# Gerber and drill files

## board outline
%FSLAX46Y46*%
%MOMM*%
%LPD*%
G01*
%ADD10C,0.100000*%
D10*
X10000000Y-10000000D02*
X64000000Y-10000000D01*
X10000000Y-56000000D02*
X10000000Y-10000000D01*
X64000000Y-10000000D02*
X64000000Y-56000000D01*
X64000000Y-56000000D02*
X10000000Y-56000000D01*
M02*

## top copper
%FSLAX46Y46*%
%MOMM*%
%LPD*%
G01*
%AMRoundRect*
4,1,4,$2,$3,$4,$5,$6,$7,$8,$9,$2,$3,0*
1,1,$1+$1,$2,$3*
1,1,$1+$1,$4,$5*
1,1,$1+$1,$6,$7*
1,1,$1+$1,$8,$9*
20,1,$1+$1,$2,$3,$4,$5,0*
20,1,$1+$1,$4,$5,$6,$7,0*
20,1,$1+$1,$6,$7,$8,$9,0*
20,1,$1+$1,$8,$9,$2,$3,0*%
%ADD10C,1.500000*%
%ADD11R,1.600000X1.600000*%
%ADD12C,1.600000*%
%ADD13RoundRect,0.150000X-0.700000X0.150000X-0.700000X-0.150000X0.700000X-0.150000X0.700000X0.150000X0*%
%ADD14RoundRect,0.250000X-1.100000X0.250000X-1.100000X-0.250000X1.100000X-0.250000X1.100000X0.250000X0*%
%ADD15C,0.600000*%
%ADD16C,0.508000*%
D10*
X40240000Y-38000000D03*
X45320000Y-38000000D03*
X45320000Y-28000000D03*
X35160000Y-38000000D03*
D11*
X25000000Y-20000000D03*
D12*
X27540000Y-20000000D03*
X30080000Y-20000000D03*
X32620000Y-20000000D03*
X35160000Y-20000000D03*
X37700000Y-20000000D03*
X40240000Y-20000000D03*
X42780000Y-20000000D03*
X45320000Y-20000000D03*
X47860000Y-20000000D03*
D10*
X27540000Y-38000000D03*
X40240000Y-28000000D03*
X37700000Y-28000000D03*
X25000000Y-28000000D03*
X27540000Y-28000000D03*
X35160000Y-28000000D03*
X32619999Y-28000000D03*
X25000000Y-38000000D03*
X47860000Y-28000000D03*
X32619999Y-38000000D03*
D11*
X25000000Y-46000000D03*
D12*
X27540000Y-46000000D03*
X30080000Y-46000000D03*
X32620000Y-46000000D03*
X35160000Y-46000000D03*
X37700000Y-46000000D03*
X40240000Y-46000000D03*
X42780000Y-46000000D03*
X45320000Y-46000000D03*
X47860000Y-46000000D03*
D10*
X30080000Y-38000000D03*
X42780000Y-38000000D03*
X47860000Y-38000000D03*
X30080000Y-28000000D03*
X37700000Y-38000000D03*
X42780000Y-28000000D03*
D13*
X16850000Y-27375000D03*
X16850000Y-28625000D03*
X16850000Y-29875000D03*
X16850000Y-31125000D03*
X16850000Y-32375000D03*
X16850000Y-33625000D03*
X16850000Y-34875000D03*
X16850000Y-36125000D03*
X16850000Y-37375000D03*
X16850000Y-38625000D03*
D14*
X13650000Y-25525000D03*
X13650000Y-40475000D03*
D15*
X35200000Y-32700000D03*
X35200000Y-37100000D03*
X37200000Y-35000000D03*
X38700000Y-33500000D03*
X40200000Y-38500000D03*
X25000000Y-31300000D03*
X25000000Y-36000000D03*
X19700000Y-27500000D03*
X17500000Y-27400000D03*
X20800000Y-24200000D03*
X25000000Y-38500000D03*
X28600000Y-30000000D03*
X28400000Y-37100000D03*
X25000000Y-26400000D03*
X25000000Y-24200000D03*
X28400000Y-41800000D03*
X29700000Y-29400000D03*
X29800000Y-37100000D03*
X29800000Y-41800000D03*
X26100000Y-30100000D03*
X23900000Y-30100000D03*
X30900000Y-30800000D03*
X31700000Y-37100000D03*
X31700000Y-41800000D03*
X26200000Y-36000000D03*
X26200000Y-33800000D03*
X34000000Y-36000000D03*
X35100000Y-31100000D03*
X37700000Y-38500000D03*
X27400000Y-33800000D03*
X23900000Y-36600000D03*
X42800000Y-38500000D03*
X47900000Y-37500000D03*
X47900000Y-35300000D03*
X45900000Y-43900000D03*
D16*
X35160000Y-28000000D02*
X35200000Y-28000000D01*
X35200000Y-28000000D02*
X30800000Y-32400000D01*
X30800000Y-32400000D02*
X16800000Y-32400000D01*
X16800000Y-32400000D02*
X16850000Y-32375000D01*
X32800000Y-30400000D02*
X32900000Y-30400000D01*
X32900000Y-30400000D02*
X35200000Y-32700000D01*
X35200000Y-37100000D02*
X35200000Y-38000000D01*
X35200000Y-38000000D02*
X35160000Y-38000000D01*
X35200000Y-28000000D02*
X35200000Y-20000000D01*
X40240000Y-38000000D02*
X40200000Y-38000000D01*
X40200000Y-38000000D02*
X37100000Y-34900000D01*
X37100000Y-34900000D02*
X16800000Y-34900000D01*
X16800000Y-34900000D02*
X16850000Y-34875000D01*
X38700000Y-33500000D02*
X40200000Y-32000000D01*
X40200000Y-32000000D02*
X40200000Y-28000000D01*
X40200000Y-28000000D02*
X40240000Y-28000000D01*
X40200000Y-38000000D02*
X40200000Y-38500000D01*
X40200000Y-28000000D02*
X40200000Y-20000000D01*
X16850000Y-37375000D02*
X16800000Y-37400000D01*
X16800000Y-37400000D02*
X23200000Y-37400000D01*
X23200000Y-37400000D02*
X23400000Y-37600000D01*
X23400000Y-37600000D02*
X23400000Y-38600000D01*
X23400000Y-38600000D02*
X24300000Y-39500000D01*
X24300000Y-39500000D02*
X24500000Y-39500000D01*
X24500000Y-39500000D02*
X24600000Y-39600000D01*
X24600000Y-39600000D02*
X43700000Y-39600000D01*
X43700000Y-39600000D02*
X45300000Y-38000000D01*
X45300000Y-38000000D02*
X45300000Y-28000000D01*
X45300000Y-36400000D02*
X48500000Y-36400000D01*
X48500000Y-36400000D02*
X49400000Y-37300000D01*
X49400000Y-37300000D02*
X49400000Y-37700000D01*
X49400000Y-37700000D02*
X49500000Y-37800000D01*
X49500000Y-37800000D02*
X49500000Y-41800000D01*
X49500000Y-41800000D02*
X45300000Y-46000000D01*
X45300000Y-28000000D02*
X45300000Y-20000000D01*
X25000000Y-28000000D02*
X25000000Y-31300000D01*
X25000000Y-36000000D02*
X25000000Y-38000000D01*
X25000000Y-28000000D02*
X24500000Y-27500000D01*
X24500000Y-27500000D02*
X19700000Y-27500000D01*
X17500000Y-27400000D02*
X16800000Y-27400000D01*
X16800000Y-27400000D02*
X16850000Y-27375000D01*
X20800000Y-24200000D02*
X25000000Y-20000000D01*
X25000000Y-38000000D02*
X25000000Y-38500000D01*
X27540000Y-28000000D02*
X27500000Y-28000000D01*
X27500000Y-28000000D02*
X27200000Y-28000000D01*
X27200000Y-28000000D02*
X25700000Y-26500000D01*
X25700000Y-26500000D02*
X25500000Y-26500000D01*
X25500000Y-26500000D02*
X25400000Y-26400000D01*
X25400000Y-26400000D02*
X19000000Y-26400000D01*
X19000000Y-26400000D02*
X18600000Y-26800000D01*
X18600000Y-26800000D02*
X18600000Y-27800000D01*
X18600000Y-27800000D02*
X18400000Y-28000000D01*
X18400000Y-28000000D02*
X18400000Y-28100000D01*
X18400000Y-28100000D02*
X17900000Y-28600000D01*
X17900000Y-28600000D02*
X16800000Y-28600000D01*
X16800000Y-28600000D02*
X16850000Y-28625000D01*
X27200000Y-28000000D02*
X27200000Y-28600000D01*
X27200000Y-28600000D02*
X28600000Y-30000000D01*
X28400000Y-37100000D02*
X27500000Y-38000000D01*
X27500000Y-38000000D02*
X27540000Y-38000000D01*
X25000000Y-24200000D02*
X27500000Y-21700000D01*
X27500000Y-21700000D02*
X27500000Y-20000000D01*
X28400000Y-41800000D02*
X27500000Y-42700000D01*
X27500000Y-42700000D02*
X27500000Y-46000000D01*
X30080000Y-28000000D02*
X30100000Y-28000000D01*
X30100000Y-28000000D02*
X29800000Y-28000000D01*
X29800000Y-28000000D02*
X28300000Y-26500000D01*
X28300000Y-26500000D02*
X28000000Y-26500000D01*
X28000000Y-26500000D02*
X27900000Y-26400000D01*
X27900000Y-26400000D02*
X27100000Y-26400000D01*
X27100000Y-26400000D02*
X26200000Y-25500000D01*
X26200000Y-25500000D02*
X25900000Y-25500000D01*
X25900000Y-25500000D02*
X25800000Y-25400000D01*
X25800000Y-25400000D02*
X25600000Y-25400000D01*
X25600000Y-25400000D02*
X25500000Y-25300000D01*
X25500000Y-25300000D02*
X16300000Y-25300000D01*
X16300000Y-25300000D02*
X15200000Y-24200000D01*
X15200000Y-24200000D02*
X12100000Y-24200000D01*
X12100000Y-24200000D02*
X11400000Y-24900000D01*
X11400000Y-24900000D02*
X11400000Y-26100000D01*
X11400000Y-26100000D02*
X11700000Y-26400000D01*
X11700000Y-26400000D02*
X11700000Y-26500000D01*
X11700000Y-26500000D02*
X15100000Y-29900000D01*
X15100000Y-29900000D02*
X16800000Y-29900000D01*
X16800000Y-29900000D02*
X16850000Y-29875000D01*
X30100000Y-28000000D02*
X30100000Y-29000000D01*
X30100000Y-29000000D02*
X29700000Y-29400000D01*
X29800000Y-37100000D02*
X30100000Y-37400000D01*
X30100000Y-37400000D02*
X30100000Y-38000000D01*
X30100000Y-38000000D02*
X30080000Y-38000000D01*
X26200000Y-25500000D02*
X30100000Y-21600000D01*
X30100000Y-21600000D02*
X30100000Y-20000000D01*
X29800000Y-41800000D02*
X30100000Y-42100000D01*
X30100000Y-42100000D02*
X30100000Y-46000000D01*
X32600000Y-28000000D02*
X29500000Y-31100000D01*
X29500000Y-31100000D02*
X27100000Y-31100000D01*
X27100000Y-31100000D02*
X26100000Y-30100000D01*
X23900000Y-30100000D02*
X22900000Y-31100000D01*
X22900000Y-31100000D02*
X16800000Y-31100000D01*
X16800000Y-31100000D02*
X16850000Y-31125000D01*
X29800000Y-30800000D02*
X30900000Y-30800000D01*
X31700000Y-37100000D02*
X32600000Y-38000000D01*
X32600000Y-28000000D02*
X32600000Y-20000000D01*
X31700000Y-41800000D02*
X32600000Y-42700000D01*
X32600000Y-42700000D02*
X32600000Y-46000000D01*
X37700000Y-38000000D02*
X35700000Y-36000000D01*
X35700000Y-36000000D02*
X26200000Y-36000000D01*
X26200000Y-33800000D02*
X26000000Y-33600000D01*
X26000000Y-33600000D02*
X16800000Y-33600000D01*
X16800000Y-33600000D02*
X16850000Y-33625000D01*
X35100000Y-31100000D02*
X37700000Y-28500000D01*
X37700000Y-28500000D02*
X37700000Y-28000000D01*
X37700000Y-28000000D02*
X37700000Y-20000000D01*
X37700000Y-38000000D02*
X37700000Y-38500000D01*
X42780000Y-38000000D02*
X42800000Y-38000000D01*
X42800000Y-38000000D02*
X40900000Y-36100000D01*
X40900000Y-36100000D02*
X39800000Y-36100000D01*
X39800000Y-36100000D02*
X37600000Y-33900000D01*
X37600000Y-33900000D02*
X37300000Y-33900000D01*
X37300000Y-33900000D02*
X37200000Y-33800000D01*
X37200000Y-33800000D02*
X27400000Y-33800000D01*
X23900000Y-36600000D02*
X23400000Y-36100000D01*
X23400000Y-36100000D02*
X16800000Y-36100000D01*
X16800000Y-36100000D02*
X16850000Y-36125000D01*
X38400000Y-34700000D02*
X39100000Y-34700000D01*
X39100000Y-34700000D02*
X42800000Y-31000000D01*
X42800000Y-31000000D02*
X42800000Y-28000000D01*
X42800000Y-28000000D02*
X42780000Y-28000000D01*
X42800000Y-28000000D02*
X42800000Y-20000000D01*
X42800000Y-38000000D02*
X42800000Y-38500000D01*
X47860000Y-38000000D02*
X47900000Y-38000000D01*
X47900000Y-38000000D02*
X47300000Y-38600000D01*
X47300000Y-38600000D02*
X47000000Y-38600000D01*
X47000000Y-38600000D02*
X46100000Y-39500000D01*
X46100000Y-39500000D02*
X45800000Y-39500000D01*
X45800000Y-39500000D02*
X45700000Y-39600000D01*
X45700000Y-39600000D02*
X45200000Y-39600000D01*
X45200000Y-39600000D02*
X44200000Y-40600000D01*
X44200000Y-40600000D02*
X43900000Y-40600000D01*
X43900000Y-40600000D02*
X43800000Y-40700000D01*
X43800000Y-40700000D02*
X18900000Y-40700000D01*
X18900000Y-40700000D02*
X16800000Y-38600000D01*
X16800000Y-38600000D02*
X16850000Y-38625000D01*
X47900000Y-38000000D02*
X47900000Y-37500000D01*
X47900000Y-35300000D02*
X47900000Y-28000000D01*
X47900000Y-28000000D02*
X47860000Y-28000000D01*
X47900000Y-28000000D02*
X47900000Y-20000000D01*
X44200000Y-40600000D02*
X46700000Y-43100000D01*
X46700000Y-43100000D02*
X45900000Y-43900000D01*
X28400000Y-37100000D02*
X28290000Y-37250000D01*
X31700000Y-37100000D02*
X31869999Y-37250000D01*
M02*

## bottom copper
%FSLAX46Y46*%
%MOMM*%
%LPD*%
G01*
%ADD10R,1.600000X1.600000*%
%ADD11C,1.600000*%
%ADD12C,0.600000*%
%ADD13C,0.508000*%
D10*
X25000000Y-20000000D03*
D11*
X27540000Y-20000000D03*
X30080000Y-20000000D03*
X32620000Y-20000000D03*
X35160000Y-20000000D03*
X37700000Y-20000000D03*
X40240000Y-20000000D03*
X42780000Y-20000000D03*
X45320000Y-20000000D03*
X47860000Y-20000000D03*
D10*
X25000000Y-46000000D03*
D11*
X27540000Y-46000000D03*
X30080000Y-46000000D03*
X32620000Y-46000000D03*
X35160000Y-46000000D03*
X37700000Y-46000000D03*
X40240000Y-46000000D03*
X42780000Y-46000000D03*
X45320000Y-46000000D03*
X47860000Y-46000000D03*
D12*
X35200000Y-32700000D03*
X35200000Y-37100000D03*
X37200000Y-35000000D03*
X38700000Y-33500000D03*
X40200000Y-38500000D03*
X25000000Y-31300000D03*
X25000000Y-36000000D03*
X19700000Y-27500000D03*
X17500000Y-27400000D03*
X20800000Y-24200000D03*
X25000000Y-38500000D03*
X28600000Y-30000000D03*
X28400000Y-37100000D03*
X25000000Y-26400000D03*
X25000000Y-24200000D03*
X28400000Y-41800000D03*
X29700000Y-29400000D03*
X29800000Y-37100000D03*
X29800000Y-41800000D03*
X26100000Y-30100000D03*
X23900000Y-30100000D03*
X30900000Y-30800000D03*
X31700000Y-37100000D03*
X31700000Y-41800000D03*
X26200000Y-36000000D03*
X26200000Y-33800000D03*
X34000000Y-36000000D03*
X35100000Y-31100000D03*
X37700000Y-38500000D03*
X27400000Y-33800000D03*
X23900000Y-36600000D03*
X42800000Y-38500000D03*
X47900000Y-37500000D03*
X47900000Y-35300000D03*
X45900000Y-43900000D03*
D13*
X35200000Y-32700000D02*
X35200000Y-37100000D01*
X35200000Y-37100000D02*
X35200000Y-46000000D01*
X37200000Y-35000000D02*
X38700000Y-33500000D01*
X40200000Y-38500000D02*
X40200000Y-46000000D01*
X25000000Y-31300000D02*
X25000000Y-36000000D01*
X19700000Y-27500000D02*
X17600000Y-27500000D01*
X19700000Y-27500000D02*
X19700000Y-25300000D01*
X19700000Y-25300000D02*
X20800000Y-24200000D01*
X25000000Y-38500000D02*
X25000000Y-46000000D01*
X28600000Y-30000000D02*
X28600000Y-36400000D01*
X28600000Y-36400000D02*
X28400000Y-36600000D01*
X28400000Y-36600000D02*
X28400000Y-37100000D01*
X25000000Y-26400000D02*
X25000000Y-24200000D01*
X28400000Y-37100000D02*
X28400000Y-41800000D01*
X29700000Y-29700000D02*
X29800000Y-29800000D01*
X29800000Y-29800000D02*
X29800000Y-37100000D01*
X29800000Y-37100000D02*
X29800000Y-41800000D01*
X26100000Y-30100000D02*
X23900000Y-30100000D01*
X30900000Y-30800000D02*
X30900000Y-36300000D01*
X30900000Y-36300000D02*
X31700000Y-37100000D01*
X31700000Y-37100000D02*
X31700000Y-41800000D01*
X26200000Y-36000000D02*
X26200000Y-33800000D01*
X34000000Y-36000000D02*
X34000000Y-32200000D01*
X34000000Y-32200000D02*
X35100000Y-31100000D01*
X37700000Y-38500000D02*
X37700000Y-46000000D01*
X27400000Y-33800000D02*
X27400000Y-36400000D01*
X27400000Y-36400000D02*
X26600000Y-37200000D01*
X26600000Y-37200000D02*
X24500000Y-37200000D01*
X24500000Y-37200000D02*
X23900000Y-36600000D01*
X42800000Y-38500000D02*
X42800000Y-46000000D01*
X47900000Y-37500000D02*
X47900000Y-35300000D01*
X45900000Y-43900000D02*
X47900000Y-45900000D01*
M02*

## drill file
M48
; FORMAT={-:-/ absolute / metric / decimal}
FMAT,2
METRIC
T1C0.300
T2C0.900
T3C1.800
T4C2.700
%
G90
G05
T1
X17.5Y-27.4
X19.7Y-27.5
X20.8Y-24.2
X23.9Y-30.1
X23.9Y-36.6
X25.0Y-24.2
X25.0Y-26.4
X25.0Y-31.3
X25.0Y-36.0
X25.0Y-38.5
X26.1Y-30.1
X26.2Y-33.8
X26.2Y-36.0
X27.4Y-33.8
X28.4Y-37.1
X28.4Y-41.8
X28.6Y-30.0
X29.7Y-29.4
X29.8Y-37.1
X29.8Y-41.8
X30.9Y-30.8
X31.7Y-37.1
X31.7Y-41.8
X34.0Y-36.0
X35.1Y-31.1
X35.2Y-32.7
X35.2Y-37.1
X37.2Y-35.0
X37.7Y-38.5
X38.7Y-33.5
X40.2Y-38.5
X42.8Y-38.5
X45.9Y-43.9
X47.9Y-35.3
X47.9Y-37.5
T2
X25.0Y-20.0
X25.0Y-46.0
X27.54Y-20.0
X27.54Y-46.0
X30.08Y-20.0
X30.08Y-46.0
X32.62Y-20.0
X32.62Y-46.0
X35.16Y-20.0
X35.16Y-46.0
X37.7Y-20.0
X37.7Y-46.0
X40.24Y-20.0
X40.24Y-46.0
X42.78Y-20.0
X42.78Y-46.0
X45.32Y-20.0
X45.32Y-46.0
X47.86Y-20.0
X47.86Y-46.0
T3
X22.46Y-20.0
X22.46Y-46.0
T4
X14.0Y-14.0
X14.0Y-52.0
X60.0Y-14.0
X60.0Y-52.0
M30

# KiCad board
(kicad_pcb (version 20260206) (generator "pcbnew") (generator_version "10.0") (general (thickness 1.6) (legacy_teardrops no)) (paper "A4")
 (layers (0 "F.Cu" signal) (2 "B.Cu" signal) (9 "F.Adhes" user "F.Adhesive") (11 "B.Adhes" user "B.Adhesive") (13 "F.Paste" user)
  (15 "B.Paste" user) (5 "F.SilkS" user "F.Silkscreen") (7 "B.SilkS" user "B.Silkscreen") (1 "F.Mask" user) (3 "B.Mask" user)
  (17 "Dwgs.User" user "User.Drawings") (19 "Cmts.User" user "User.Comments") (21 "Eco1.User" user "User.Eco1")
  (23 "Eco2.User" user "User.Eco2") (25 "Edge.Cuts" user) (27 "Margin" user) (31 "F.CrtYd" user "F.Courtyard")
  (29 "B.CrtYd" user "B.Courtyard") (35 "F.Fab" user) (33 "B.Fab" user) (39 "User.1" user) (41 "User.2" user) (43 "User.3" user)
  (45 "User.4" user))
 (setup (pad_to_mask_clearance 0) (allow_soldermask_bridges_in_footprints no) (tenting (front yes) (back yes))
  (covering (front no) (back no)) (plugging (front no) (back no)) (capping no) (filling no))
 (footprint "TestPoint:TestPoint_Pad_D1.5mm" (layer "F.Cu") (at 40.24 38)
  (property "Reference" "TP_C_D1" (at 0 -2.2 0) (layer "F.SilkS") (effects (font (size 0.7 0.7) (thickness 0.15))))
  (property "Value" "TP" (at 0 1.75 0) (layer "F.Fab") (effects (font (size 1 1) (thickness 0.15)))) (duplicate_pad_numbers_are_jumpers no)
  (pad "1" smd circle (at 0 0) (size 1.5 1.5) (layers "F.Cu" "F.Mask") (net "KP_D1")))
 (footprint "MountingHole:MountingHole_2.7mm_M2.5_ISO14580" (layer "F.Cu") (at 60 14)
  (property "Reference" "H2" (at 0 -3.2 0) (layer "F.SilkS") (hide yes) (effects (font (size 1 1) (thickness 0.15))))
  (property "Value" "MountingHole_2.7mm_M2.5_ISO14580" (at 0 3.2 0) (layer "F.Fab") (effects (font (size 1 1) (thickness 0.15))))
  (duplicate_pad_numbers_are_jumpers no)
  (pad "" np_thru_hole circle (at 0 0) (size 2.7 2.7) (drill 2.7) (layers "*.Cu" "*.Mask")))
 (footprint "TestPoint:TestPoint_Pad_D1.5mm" (layer "F.Cu") (at 45.32 38)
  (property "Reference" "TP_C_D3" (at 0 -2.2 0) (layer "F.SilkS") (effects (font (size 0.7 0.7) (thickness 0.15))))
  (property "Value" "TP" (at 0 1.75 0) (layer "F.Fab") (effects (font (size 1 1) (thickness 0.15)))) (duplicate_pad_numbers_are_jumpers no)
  (pad "1" smd circle (at 0 0) (size 1.5 1.5) (layers "F.Cu" "F.Mask") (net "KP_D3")))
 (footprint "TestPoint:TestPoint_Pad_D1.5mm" (layer "F.Cu") (at 45.32 28)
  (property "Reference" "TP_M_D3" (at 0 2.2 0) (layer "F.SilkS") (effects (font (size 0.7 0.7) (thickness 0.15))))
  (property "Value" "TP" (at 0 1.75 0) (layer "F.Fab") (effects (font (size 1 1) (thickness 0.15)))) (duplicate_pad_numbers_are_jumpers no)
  (pad "1" smd circle (at 0 0) (size 1.5 1.5) (layers "F.Cu" "F.Mask") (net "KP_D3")))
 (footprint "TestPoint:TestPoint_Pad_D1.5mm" (layer "F.Cu") (at 35.16 38)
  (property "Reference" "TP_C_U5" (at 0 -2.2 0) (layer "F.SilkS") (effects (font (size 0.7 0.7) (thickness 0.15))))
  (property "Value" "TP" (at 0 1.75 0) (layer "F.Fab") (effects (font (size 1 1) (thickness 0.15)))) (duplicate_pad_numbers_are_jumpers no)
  (pad "1" smd circle (at 0 0) (size 1.5 1.5) (layers "F.Cu" "F.Mask") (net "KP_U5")))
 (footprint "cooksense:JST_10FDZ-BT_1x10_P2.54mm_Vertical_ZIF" (layer "F.Cu") (at 25 20)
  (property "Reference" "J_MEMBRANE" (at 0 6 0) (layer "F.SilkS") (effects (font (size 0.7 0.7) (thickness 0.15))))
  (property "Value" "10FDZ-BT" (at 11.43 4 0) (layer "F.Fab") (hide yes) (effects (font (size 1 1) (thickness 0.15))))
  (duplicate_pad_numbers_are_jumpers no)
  (pad "" np_thru_hole circle (at -2.54 0) (size 1.8 1.8) (drill 1.8) (layers "*.Cu" "*.Mask"))
  (pad "1" thru_hole rect (at 0 0) (size 1.6 1.6) (drill 0.9) (layers "*.Cu" "*.Mask") (remove_unused_layers no) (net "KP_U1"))
  (pad "2" thru_hole circle (at 2.54 0) (size 1.6 1.6) (drill 0.9) (layers "*.Cu" "*.Mask") (remove_unused_layers no) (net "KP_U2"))
  (pad "3" thru_hole circle (at 5.08 0) (size 1.6 1.6) (drill 0.9) (layers "*.Cu" "*.Mask") (remove_unused_layers no) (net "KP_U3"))
  (pad "4" thru_hole circle (at 7.62 0) (size 1.6 1.6) (drill 0.9) (layers "*.Cu" "*.Mask") (remove_unused_layers no) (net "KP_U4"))
  (pad "5" thru_hole circle (at 10.16 0) (size 1.6 1.6) (drill 0.9) (layers "*.Cu" "*.Mask") (remove_unused_layers no) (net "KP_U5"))
  (pad "6" thru_hole circle (at 12.7 0) (size 1.6 1.6) (drill 0.9) (layers "*.Cu" "*.Mask") (remove_unused_layers no) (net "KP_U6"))
  (pad "7" thru_hole circle (at 15.24 0) (size 1.6 1.6) (drill 0.9) (layers "*.Cu" "*.Mask") (remove_unused_layers no) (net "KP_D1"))
  (pad "8" thru_hole circle (at 17.78 0) (size 1.6 1.6) (drill 0.9) (layers "*.Cu" "*.Mask") (remove_unused_layers no) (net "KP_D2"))
  (pad "9" thru_hole circle (at 20.32 0) (size 1.6 1.6) (drill 0.9) (layers "*.Cu" "*.Mask") (remove_unused_layers no) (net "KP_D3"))
  (pad "10" thru_hole circle (at 22.86 0) (size 1.6 1.6) (drill 0.9) (layers "*.Cu" "*.Mask") (remove_unused_layers no) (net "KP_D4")))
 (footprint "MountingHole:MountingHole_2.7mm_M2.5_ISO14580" (layer "F.Cu") (at 14 14)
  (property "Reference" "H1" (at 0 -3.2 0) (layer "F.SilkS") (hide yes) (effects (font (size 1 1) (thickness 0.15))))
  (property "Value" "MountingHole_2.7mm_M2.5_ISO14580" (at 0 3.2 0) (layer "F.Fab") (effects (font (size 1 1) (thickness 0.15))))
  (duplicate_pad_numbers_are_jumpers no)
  (pad "" np_thru_hole circle (at 0 0) (size 2.7 2.7) (drill 2.7) (layers "*.Cu" "*.Mask")))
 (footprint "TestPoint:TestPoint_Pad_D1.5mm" (layer "F.Cu") (at 27.54 38)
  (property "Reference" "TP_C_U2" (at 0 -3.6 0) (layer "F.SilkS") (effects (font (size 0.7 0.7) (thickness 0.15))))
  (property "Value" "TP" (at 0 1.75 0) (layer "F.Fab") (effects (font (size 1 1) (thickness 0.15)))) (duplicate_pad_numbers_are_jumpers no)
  (pad "1" smd circle (at 0 0) (size 1.5 1.5) (layers "F.Cu" "F.Mask") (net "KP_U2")))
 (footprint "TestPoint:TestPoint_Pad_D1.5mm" (layer "F.Cu") (at 40.24 28)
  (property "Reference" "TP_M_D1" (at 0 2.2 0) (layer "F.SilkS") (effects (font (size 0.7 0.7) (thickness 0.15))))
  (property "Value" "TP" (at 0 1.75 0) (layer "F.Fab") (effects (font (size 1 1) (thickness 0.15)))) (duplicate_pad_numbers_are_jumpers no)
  (pad "1" smd circle (at 0 0) (size 1.5 1.5) (layers "F.Cu" "F.Mask") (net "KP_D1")))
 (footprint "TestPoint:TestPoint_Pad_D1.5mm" (layer "F.Cu") (at 37.7 28)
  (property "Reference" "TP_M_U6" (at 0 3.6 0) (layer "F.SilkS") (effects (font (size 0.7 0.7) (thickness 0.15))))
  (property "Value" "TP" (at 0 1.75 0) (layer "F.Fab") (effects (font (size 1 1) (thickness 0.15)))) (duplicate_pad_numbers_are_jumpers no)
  (pad "1" smd circle (at 0 0) (size 1.5 1.5) (layers "F.Cu" "F.Mask") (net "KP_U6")))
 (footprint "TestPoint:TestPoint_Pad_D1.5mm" (layer "F.Cu") (at 25 28)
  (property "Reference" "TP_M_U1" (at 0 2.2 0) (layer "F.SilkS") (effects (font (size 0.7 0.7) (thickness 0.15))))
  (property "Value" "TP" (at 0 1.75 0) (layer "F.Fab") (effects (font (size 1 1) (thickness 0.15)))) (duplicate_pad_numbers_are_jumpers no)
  (pad "1" smd circle (at 0 0) (size 1.5 1.5) (layers "F.Cu" "F.Mask") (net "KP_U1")))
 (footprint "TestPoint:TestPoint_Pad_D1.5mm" (layer "F.Cu") (at 27.54 28)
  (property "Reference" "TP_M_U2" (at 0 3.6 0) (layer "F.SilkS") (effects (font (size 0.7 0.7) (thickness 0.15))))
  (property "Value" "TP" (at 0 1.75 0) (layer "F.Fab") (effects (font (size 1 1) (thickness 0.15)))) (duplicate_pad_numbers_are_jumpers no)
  (pad "1" smd circle (at 0 0) (size 1.5 1.5) (layers "F.Cu" "F.Mask") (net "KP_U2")))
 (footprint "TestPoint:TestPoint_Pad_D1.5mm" (layer "F.Cu") (at 35.16 28)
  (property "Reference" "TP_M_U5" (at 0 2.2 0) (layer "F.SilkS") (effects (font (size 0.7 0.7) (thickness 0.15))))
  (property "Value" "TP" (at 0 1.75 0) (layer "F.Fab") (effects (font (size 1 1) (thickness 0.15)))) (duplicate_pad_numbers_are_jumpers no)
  (pad "1" smd circle (at 0 0) (size 1.5 1.5) (layers "F.Cu" "F.Mask") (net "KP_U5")))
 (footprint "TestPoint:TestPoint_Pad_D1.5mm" (layer "F.Cu") (at 32.619999 28)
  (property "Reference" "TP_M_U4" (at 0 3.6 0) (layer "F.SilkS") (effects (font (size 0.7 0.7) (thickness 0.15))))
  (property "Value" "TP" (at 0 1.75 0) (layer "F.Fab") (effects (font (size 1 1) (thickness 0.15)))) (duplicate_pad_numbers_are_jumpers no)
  (pad "1" smd circle (at 0 0) (size 1.5 1.5) (layers "F.Cu" "F.Mask") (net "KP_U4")))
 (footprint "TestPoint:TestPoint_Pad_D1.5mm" (layer "F.Cu") (at 25 38)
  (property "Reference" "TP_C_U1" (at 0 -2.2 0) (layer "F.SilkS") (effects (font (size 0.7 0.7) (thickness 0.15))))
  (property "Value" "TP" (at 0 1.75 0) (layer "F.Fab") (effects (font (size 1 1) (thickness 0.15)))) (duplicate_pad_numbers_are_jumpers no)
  (pad "1" smd circle (at 0 0) (size 1.5 1.5) (layers "F.Cu" "F.Mask") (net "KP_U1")))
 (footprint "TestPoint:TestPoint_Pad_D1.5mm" (layer "F.Cu") (at 47.86 28)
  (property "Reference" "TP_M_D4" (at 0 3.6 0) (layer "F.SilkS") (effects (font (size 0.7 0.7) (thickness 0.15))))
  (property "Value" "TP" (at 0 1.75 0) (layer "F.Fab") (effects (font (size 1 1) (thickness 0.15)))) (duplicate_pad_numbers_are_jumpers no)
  (pad "1" smd circle (at 0 0) (size 1.5 1.5) (layers "F.Cu" "F.Mask") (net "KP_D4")))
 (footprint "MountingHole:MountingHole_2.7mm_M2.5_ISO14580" (layer "F.Cu") (at 60 52)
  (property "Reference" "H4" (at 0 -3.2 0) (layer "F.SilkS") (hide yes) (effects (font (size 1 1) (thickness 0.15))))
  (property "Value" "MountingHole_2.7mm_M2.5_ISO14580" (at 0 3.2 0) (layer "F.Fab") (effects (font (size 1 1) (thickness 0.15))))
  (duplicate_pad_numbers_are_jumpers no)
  (pad "" np_thru_hole circle (at 0 0) (size 2.7 2.7) (drill 2.7) (layers "*.Cu" "*.Mask")))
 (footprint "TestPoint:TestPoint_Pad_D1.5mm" (layer "F.Cu") (at 32.619999 38)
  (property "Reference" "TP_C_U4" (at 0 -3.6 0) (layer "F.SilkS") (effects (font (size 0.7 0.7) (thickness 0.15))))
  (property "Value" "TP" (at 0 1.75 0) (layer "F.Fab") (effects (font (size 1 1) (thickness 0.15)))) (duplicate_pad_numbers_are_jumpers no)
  (pad "1" smd circle (at 0 0) (size 1.5 1.5) (layers "F.Cu" "F.Mask") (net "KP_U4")))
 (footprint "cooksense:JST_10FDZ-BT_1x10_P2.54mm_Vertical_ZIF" (layer "F.Cu") (at 25 46)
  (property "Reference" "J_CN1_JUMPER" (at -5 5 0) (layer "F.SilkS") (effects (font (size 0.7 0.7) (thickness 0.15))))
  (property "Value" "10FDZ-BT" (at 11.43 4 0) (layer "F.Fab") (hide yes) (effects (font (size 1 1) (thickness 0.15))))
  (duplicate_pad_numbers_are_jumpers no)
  (pad "" np_thru_hole circle (at -2.54 0) (size 1.8 1.8) (drill 1.8) (layers "*.Cu" "*.Mask"))
  (pad "1" thru_hole rect (at 0 0) (size 1.6 1.6) (drill 0.9) (layers "*.Cu" "*.Mask") (remove_unused_layers no) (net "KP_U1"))
  (pad "2" thru_hole circle (at 2.54 0) (size 1.6 1.6) (drill 0.9) (layers "*.Cu" "*.Mask") (remove_unused_layers no) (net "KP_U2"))
  (pad "3" thru_hole circle (at 5.08 0) (size 1.6 1.6) (drill 0.9) (layers "*.Cu" "*.Mask") (remove_unused_layers no) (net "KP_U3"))
  (pad "4" thru_hole circle (at 7.62 0) (size 1.6 1.6) (drill 0.9) (layers "*.Cu" "*.Mask") (remove_unused_layers no) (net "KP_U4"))
  (pad "5" thru_hole circle (at 10.16 0) (size 1.6 1.6) (drill 0.9) (layers "*.Cu" "*.Mask") (remove_unused_layers no) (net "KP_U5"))
  (pad "6" thru_hole circle (at 12.7 0) (size 1.6 1.6) (drill 0.9) (layers "*.Cu" "*.Mask") (remove_unused_layers no) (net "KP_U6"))
  (pad "7" thru_hole circle (at 15.24 0) (size 1.6 1.6) (drill 0.9) (layers "*.Cu" "*.Mask") (remove_unused_layers no) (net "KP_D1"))
  (pad "8" thru_hole circle (at 17.78 0) (size 1.6 1.6) (drill 0.9) (layers "*.Cu" "*.Mask") (remove_unused_layers no) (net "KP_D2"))
  (pad "9" thru_hole circle (at 20.32 0) (size 1.6 1.6) (drill 0.9) (layers "*.Cu" "*.Mask") (remove_unused_layers no) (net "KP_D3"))
  (pad "10" thru_hole circle (at 22.86 0) (size 1.6 1.6) (drill 0.9) (layers "*.Cu" "*.Mask") (remove_unused_layers no) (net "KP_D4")))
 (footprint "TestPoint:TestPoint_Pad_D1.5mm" (layer "F.Cu") (at 30.08 38)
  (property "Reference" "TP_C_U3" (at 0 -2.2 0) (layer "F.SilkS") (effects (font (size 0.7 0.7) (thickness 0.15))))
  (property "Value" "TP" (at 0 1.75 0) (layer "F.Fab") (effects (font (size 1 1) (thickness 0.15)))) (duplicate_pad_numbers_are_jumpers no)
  (pad "1" smd circle (at 0 0) (size 1.5 1.5) (layers "F.Cu" "F.Mask") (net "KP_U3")))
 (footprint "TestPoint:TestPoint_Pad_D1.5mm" (layer "F.Cu") (at 42.78 38)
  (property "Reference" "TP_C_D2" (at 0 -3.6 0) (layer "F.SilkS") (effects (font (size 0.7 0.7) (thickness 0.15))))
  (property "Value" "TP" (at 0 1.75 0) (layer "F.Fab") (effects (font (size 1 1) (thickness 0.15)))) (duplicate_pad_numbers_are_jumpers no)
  (pad "1" smd circle (at 0 0) (size 1.5 1.5) (layers "F.Cu" "F.Mask") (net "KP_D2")))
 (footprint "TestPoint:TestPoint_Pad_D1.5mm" (layer "F.Cu") (at 47.86 38)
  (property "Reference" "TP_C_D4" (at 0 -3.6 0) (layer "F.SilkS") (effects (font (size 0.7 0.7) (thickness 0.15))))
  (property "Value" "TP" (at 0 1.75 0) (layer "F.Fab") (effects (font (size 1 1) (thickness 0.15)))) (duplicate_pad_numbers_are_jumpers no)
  (pad "1" smd circle (at 0 0) (size 1.5 1.5) (layers "F.Cu" "F.Mask") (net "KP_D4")))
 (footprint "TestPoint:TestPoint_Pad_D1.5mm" (layer "F.Cu") (at 30.08 28)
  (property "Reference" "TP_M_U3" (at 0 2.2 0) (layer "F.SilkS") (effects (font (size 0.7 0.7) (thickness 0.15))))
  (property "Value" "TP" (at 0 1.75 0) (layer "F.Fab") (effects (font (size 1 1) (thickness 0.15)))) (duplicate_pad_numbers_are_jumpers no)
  (pad "1" smd circle (at 0 0) (size 1.5 1.5) (layers "F.Cu" "F.Mask") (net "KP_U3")))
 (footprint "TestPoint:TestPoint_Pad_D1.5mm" (layer "F.Cu") (at 37.7 38)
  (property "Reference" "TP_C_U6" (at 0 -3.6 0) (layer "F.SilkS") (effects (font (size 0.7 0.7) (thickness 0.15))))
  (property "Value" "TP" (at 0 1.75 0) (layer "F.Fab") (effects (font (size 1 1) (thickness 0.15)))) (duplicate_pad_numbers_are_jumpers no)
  (pad "1" smd circle (at 0 0) (size 1.5 1.5) (layers "F.Cu" "F.Mask") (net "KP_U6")))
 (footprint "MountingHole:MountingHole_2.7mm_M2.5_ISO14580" (layer "F.Cu") (at 14 52)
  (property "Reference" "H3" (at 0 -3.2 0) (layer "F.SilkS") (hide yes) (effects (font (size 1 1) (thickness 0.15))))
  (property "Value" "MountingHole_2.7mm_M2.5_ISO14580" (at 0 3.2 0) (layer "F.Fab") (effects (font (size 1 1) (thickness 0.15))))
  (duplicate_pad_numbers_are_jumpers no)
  (pad "" np_thru_hole circle (at 0 0) (size 2.7 2.7) (drill 2.7) (layers "*.Cu" "*.Mask")))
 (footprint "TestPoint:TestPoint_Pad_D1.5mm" (layer "F.Cu") (at 42.78 28)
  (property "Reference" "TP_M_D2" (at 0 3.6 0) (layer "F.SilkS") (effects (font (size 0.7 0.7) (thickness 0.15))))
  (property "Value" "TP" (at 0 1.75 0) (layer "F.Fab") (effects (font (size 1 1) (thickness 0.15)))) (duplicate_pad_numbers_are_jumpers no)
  (pad "1" smd circle (at 0 0) (size 1.5 1.5) (layers "F.Cu" "F.Mask") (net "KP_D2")))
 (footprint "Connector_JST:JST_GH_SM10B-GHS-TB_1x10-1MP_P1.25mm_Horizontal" (layer "F.Cu") (at 15 33 -90)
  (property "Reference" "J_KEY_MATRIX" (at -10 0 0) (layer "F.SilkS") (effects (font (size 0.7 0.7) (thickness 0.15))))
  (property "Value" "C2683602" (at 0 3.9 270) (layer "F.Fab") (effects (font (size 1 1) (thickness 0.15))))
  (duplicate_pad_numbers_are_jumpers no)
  (pad "1" smd roundrect (at -5.625 -1.85 270) (size 0.6 1.7) (layers "F.Cu" "F.Mask" "F.Paste") (roundrect_rratio 0.25) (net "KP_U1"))
  (pad "2" smd roundrect (at -4.375 -1.85 270) (size 0.6 1.7) (layers "F.Cu" "F.Mask" "F.Paste") (roundrect_rratio 0.25) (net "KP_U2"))
  (pad "3" smd roundrect (at -3.125 -1.85 270) (size 0.6 1.7) (layers "F.Cu" "F.Mask" "F.Paste") (roundrect_rratio 0.25) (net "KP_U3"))
  (pad "4" smd roundrect (at -1.875 -1.85 270) (size 0.6 1.7) (layers "F.Cu" "F.Mask" "F.Paste") (roundrect_rratio 0.25) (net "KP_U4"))
  (pad "5" smd roundrect (at -0.625 -1.85 270) (size 0.6 1.7) (layers "F.Cu" "F.Mask" "F.Paste") (roundrect_rratio 0.25) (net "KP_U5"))
  (pad "6" smd roundrect (at 0.625 -1.85 270) (size 0.6 1.7) (layers "F.Cu" "F.Mask" "F.Paste") (roundrect_rratio 0.25) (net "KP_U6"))
  (pad "7" smd roundrect (at 1.875 -1.85 270) (size 0.6 1.7) (layers "F.Cu" "F.Mask" "F.Paste") (roundrect_rratio 0.25) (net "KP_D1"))
  (pad "8" smd roundrect (at 3.125 -1.85 270) (size 0.6 1.7) (layers "F.Cu" "F.Mask" "F.Paste") (roundrect_rratio 0.25) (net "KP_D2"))
  (pad "9" smd roundrect (at 4.375 -1.85 270) (size 0.6 1.7) (layers "F.Cu" "F.Mask" "F.Paste") (roundrect_rratio 0.25) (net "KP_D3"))
  (pad "10" smd roundrect (at 5.625 -1.85 270) (size 0.6 1.7) (layers "F.Cu" "F.Mask" "F.Paste") (roundrect_rratio 0.25) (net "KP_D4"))
  (pad "MP" smd roundrect (at -7.475 1.35 270) (size 1 2.7) (layers "F.Cu" "F.Mask" "F.Paste") (roundrect_rratio 0.25))
  (pad "MP" smd roundrect (at 7.475 1.35 270) (size 1 2.7) (layers "F.Cu" "F.Mask" "F.Paste") (roundrect_rratio 0.25)))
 (gr_line (start 10 10) (end 64 10) (stroke (width 0.1) (type default)) (layer "Edge.Cuts"))
 (gr_line (start 10 56) (end 10 10) (stroke (width 0.1) (type default)) (layer "Edge.Cuts"))
 (gr_line (start 64 10) (end 64 56) (stroke (width 0.1) (type default)) (layer "Edge.Cuts"))
 (gr_line (start 64 56) (end 10 56) (stroke (width 0.1) (type default)) (layer "Edge.Cuts"))
 (segment (start 35.160000 28.000000) (end 35.200000 28.000000) (width 0.508) (layer "F.Cu") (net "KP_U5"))
 (segment (start 35.200000 28.000000) (end 30.800000 32.400000) (width 0.508) (layer "F.Cu") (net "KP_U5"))
 (segment (start 30.800000 32.400000) (end 16.800000 32.400000) (width 0.508) (layer "F.Cu") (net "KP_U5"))
 (segment (start 16.800000 32.400000) (end 16.850000 32.375000) (width 0.508) (layer "F.Cu") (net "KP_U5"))
 (segment (start 32.800000 30.400000) (end 32.900000 30.400000) (width 0.508) (layer "F.Cu") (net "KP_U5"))
 (segment (start 32.900000 30.400000) (end 35.200000 32.700000) (width 0.508) (layer "F.Cu") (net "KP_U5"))
 (segment (start 35.200000 32.700000) (end 35.200000 37.100000) (width 0.508) (layer "B.Cu") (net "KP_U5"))
 (segment (start 35.200000 37.100000) (end 35.200000 38.000000) (width 0.508) (layer "F.Cu") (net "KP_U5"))
 (segment (start 35.200000 38.000000) (end 35.160000 38.000000) (width 0.508) (layer "F.Cu") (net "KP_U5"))
 (segment (start 35.200000 37.100000) (end 35.200000 46.000000) (width 0.508) (layer "B.Cu") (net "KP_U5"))
 (segment (start 35.200000 28.000000) (end 35.200000 20.000000) (width 0.508) (layer "F.Cu") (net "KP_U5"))
 (via (at 35.200000 32.700000) (size 0.6) (drill 0.3) (layers "F.Cu" "B.Cu") (tenting (front yes) (back yes)) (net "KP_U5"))
 (via (at 35.200000 37.100000) (size 0.6) (drill 0.3) (layers "F.Cu" "B.Cu") (tenting (front yes) (back yes)) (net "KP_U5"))
 (segment (start 40.240000 38.000000) (end 40.200000 38.000000) (width 0.508) (layer "F.Cu") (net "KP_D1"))
 (segment (start 40.200000 38.000000) (end 37.100000 34.900000) (width 0.508) (layer "F.Cu") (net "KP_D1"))
 (segment (start 37.100000 34.900000) (end 16.800000 34.900000) (width 0.508) (layer "F.Cu") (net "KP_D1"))
 (segment (start 16.800000 34.900000) (end 16.850000 34.875000) (width 0.508) (layer "F.Cu") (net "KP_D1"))
 (segment (start 37.200000 35.000000) (end 38.700000 33.500000) (width 0.508) (layer "B.Cu") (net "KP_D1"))
 (segment (start 38.700000 33.500000) (end 40.200000 32.000000) (width 0.508) (layer "F.Cu") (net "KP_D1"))
 (segment (start 40.200000 32.000000) (end 40.200000 28.000000) (width 0.508) (layer "F.Cu") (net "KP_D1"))
 (segment (start 40.200000 28.000000) (end 40.240000 28.000000) (width 0.508) (layer "F.Cu") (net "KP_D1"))
 (segment (start 40.200000 38.000000) (end 40.200000 38.500000) (width 0.508) (layer "F.Cu") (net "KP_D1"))
 (segment (start 40.200000 38.500000) (end 40.200000 46.000000) (width 0.508) (layer "B.Cu") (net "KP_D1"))
 (segment (start 40.200000 28.000000) (end 40.200000 20.000000) (width 0.508) (layer "F.Cu") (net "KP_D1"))
 (via (at 37.200000 35.000000) (size 0.6) (drill 0.3) (layers "F.Cu" "B.Cu") (tenting (front yes) (back yes)) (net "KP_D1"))
 (via (at 38.700000 33.500000) (size 0.6) (drill 0.3) (layers "F.Cu" "B.Cu") (tenting (front yes) (back yes)) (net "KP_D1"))
 (via (at 40.200000 38.500000) (size 0.6) (drill 0.3) (layers "F.Cu" "B.Cu") (tenting (front yes) (back yes)) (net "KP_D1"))
 (segment (start 16.850000 37.375000) (end 16.800000 37.400000) (width 0.508) (layer "F.Cu") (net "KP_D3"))
 (segment (start 16.800000 37.400000) (end 23.200000 37.400000) (width 0.508) (layer "F.Cu") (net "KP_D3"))
 (segment (start 23.200000 37.400000) (end 23.400000 37.600000) (width 0.508) (layer "F.Cu") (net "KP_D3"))
 (segment (start 23.400000 37.600000) (end 23.400000 38.600000) (width 0.508) (layer "F.Cu") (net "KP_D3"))
 (segment (start 23.400000 38.600000) (end 24.300000 39.500000) (width 0.508) (layer "F.Cu") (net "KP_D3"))
 (segment (start 24.300000 39.500000) (end 24.500000 39.500000) (width 0.508) (layer "F.Cu") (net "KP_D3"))
 (segment (start 24.500000 39.500000) (end 24.600000 39.600000) (width 0.508) (layer "F.Cu") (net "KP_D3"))
 (segment (start 24.600000 39.600000) (end 43.700000 39.600000) (width 0.508) (layer "F.Cu") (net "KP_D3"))
 (segment (start 43.700000 39.600000) (end 45.300000 38.000000) (width 0.508) (layer "F.Cu") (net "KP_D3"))
 (segment (start 45.300000 38.000000) (end 45.300000 28.000000) (width 0.508) (layer "F.Cu") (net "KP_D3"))
 (segment (start 45.300000 36.400000) (end 48.500000 36.400000) (width 0.508) (layer "F.Cu") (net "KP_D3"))
 (segment (start 48.500000 36.400000) (end 49.400000 37.300000) (width 0.508) (layer "F.Cu") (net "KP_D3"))
 (segment (start 49.400000 37.300000) (end 49.400000 37.700000) (width 0.508) (layer "F.Cu") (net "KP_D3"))
 (segment (start 49.400000 37.700000) (end 49.500000 37.800000) (width 0.508) (layer "F.Cu") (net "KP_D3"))
 (segment (start 49.500000 37.800000) (end 49.500000 41.800000) (width 0.508) (layer "F.Cu") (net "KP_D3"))
 (segment (start 49.500000 41.800000) (end 45.300000 46.000000) (width 0.508) (layer "F.Cu") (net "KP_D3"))
 (segment (start 45.300000 28.000000) (end 45.300000 20.000000) (width 0.508) (layer "F.Cu") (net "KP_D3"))
 (segment (start 25.000000 28.000000) (end 25.000000 31.300000) (width 0.508) (layer "F.Cu") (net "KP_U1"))
 (segment (start 25.000000 31.300000) (end 25.000000 36.000000) (width 0.508) (layer "B.Cu") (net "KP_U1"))
 (segment (start 25.000000 36.000000) (end 25.000000 38.000000) (width 0.508) (layer "F.Cu") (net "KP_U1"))
 (segment (start 25.000000 28.000000) (end 24.500000 27.500000) (width 0.508) (layer "F.Cu") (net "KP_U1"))
 (segment (start 24.500000 27.500000) (end 19.700000 27.500000) (width 0.508) (layer "F.Cu") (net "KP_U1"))
 (segment (start 19.700000 27.500000) (end 17.600000 27.500000) (width 0.508) (layer "B.Cu") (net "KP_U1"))
 (segment (start 17.500000 27.400000) (end 16.800000 27.400000) (width 0.508) (layer "F.Cu") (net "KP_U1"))
 (segment (start 16.800000 27.400000) (end 16.850000 27.375000) (width 0.508) (layer "F.Cu") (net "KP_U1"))
 (segment (start 19.700000 27.500000) (end 19.700000 25.300000) (width 0.508) (layer "B.Cu") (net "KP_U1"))
 (segment (start 19.700000 25.300000) (end 20.800000 24.200000) (width 0.508) (layer "B.Cu") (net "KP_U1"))
 (segment (start 20.800000 24.200000) (end 25.000000 20.000000) (width 0.508) (layer "F.Cu") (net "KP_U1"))
 (segment (start 25.000000 38.000000) (end 25.000000 38.500000) (width 0.508) (layer "F.Cu") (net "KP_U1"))
 (segment (start 25.000000 38.500000) (end 25.000000 46.000000) (width 0.508) (layer "B.Cu") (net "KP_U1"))
 (via (at 25.000000 31.300000) (size 0.6) (drill 0.3) (layers "F.Cu" "B.Cu") (tenting (front yes) (back yes)) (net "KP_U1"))
 (via (at 25.000000 36.000000) (size 0.6) (drill 0.3) (layers "F.Cu" "B.Cu") (tenting (front yes) (back yes)) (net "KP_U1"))
 (via (at 19.700000 27.500000) (size 0.6) (drill 0.3) (layers "F.Cu" "B.Cu") (tenting (front yes) (back yes)) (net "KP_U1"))
 (via (at 17.500000 27.400000) (size 0.6) (drill 0.3) (layers "F.Cu" "B.Cu") (tenting (front yes) (back yes)) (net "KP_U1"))
 (via (at 20.800000 24.200000) (size 0.6) (drill 0.3) (layers "F.Cu" "B.Cu") (tenting (front yes) (back yes)) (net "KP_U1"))
 (via (at 25.000000 38.500000) (size 0.6) (drill 0.3) (layers "F.Cu" "B.Cu") (tenting (front yes) (back yes)) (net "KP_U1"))
 (segment (start 27.540000 28.000000) (end 27.500000 28.000000) (width 0.508) (layer "F.Cu") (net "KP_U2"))
 (segment (start 27.500000 28.000000) (end 27.200000 28.000000) (width 0.508) (layer "F.Cu") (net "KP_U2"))
 (segment (start 27.200000 28.000000) (end 25.700000 26.500000) (width 0.508) (layer "F.Cu") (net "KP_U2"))
 (segment (start 25.700000 26.500000) (end 25.500000 26.500000) (width 0.508) (layer "F.Cu") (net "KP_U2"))
 (segment (start 25.500000 26.500000) (end 25.400000 26.400000) (width 0.508) (layer "F.Cu") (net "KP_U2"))
 (segment (start 25.400000 26.400000) (end 19.000000 26.400000) (width 0.508) (layer "F.Cu") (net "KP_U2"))
 (segment (start 19.000000 26.400000) (end 18.600000 26.800000) (width 0.508) (layer "F.Cu") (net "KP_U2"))
 (segment (start 18.600000 26.800000) (end 18.600000 27.800000) (width 0.508) (layer "F.Cu") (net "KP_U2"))
 (segment (start 18.600000 27.800000) (end 18.400000 28.000000) (width 0.508) (layer "F.Cu") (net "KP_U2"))
 (segment (start 18.400000 28.000000) (end 18.400000 28.100000) (width 0.508) (layer "F.Cu") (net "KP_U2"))
 (segment (start 18.400000 28.100000) (end 17.900000 28.600000) (width 0.508) (layer "F.Cu") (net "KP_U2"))
 (segment (start 17.900000 28.600000) (end 16.800000 28.600000) (width 0.508) (layer "F.Cu") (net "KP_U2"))
 (segment (start 16.800000 28.600000) (end 16.850000 28.625000) (width 0.508) (layer "F.Cu") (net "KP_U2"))
 (segment (start 27.200000 28.000000) (end 27.200000 28.600000) (width 0.508) (layer "F.Cu") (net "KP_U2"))
 (segment (start 27.200000 28.600000) (end 28.600000 30.000000) (width 0.508) (layer "F.Cu") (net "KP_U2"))
 (segment (start 28.600000 30.000000) (end 28.600000 36.400000) (width 0.508) (layer "B.Cu") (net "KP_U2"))
 (segment (start 28.600000 36.400000) (end 28.400000 36.600000) (width 0.508) (layer "B.Cu") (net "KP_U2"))
 (segment (start 28.400000 36.600000) (end 28.400000 37.100000) (width 0.508) (layer "B.Cu") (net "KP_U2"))
 (segment (start 28.400000 37.100000) (end 27.500000 38.000000) (width 0.508) (layer "F.Cu") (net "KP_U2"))
 (segment (start 27.500000 38.000000) (end 27.540000 38.000000) (width 0.508) (layer "F.Cu") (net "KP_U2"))
 (segment (start 25.000000 26.400000) (end 25.000000 24.200000) (width 0.508) (layer "B.Cu") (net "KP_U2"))
 (segment (start 25.000000 24.200000) (end 27.500000 21.700000) (width 0.508) (layer "F.Cu") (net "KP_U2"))
 (segment (start 27.500000 21.700000) (end 27.500000 20.000000) (width 0.508) (layer "F.Cu") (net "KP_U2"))
 (segment (start 28.400000 37.100000) (end 28.400000 41.800000) (width 0.508) (layer "B.Cu") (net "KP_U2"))
 (segment (start 28.400000 41.800000) (end 27.500000 42.700000) (width 0.508) (layer "F.Cu") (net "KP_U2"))
 (segment (start 27.500000 42.700000) (end 27.500000 46.000000) (width 0.508) (layer "F.Cu") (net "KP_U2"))
 (via (at 28.600000 30.000000) (size 0.6) (drill 0.3) (layers "F.Cu" "B.Cu") (tenting (front yes) (back yes)) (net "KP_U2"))
 (via (at 28.400000 37.100000) (size 0.6) (drill 0.3) (layers "F.Cu" "B.Cu") (tenting (front yes) (back yes)) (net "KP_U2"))
 (via (at 25.000000 26.400000) (size 0.6) (drill 0.3) (layers "F.Cu" "B.Cu") (tenting (front yes) (back yes)) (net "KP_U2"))
 (via (at 25.000000 24.200000) (size 0.6) (drill 0.3) (layers "F.Cu" "B.Cu") (tenting (front yes) (back yes)) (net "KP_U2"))
 (via (at 28.400000 41.800000) (size 0.6) (drill 0.3) (layers "F.Cu" "B.Cu") (tenting (front yes) (back yes)) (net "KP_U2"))
 (segment (start 30.080000 28.000000) (end 30.100000 28.000000) (width 0.508) (layer "F.Cu") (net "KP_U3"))
 (segment (start 30.100000 28.000000) (end 29.800000 28.000000) (width 0.508) (layer "F.Cu") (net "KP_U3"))
 (segment (start 29.800000 28.000000) (end 28.300000 26.500000) (width 0.508) (layer "F.Cu") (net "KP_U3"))
 (segment (start 28.300000 26.500000) (end 28.000000 26.500000) (width 0.508) (layer "F.Cu") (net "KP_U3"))
 (segment (start 28.000000 26.500000) (end 27.900000 26.400000) (width 0.508) (layer "F.Cu") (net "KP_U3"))
 (segment (start 27.900000 26.400000) (end 27.100000 26.400000) (width 0.508) (layer "F.Cu") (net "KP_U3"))
 (segment (start 27.100000 26.400000) (end 26.200000 25.500000) (width 0.508) (layer "F.Cu") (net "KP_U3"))
 (segment (start 26.200000 25.500000) (end 25.900000 25.500000) (width 0.508) (layer "F.Cu") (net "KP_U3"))
 (segment (start 25.900000 25.500000) (end 25.800000 25.400000) (width 0.508) (layer "F.Cu") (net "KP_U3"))
 (segment (start 25.800000 25.400000) (end 25.600000 25.400000) (width 0.508) (layer "F.Cu") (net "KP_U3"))
 (segment (start 25.600000 25.400000) (end 25.500000 25.300000) (width 0.508) (layer "F.Cu") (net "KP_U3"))
 (segment (start 25.500000 25.300000) (end 16.300000 25.300000) (width 0.508) (layer "F.Cu") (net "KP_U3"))
 (segment (start 16.300000 25.300000) (end 15.200000 24.200000) (width 0.508) (layer "F.Cu") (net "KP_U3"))
 (segment (start 15.200000 24.200000) (end 12.100000 24.200000) (width 0.508) (layer "F.Cu") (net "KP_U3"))
 (segment (start 12.100000 24.200000) (end 11.400000 24.900000) (width 0.508) (layer "F.Cu") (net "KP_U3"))
 (segment (start 11.400000 24.900000) (end 11.400000 26.100000) (width 0.508) (layer "F.Cu") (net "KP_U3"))
 (segment (start 11.400000 26.100000) (end 11.700000 26.400000) (width 0.508) (layer "F.Cu") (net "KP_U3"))
 (segment (start 11.700000 26.400000) (end 11.700000 26.500000) (width 0.508) (layer "F.Cu") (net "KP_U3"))
 (segment (start 11.700000 26.500000) (end 15.100000 29.900000) (width 0.508) (layer "F.Cu") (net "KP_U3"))
 (segment (start 15.100000 29.900000) (end 16.800000 29.900000) (width 0.508) (layer "F.Cu") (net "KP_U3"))
 (segment (start 16.800000 29.900000) (end 16.850000 29.875000) (width 0.508) (layer "F.Cu") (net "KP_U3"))
 (segment (start 30.100000 28.000000) (end 30.100000 29.000000) (width 0.508) (layer "F.Cu") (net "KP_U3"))
 (segment (start 30.100000 29.000000) (end 29.700000 29.400000) (width 0.508) (layer "F.Cu") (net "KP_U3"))
 (segment (start 29.700000 29.700000) (end 29.800000 29.800000) (width 0.508) (layer "B.Cu") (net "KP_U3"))
 (segment (start 29.800000 29.800000) (end 29.800000 37.100000) (width 0.508) (layer "B.Cu") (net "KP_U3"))
 (segment (start 29.800000 37.100000) (end 30.100000 37.400000) (width 0.508) (layer "F.Cu") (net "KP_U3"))
 (segment (start 30.100000 37.400000) (end 30.100000 38.000000) (width 0.508) (layer "F.Cu") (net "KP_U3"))
 (segment (start 30.100000 38.000000) (end 30.080000 38.000000) (width 0.508) (layer "F.Cu") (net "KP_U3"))
 (segment (start 26.200000 25.500000) (end 30.100000 21.600000) (width 0.508) (layer "F.Cu") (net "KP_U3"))
 (segment (start 30.100000 21.600000) (end 30.100000 20.000000) (width 0.508) (layer "F.Cu") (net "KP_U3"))
 (segment (start 29.800000 37.100000) (end 29.800000 41.800000) (width 0.508) (layer "B.Cu") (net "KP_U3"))
 (segment (start 29.800000 41.800000) (end 30.100000 42.100000) (width 0.508) (layer "F.Cu") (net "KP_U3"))
 (segment (start 30.100000 42.100000) (end 30.100000 46.000000) (width 0.508) (layer "F.Cu") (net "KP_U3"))
 (via (at 29.700000 29.400000) (size 0.6) (drill 0.3) (layers "F.Cu" "B.Cu") (tenting (front yes) (back yes)) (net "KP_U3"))
 (via (at 29.800000 37.100000) (size 0.6) (drill 0.3) (layers "F.Cu" "B.Cu") (tenting (front yes) (back yes)) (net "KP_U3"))
 (via (at 29.800000 41.800000) (size 0.6) (drill 0.3) (layers "F.Cu" "B.Cu") (tenting (front yes) (back yes)) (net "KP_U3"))
 (segment (start 32.600000 28.000000) (end 29.500000 31.100000) (width 0.508) (layer "F.Cu") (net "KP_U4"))
 (segment (start 29.500000 31.100000) (end 27.100000 31.100000) (width 0.508) (layer "F.Cu") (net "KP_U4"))
 (segment (start 27.100000 31.100000) (end 26.100000 30.100000) (width 0.508) (layer "F.Cu") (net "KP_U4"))
 (segment (start 26.100000 30.100000) (end 23.900000 30.100000) (width 0.508) (layer "B.Cu") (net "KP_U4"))
 (segment (start 23.900000 30.100000) (end 22.900000 31.100000) (width 0.508) (layer "F.Cu") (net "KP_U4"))
 (segment (start 22.900000 31.100000) (end 16.800000 31.100000) (width 0.508) (layer "F.Cu") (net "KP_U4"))
 (segment (start 16.800000 31.100000) (end 16.850000 31.125000) (width 0.508) (layer "F.Cu") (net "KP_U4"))
 (segment (start 29.800000 30.800000) (end 30.900000 30.800000) (width 0.508) (layer "F.Cu") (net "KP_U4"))
 (segment (start 30.900000 30.800000) (end 30.900000 36.300000) (width 0.508) (layer "B.Cu") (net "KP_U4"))
 (segment (start 30.900000 36.300000) (end 31.700000 37.100000) (width 0.508) (layer "B.Cu") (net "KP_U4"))
 (segment (start 31.700000 37.100000) (end 32.600000 38.000000) (width 0.508) (layer "F.Cu") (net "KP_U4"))
 (segment (start 32.600000 28.000000) (end 32.600000 20.000000) (width 0.508) (layer "F.Cu") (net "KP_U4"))
 (segment (start 31.700000 37.100000) (end 31.700000 41.800000) (width 0.508) (layer "B.Cu") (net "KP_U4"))
 (segment (start 31.700000 41.800000) (end 32.600000 42.700000) (width 0.508) (layer "F.Cu") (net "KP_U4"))
 (segment (start 32.600000 42.700000) (end 32.600000 46.000000) (width 0.508) (layer "F.Cu") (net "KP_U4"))
 (via (at 26.100000 30.100000) (size 0.6) (drill 0.3) (layers "F.Cu" "B.Cu") (tenting (front yes) (back yes)) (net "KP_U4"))
 (via (at 23.900000 30.100000) (size 0.6) (drill 0.3) (layers "F.Cu" "B.Cu") (tenting (front yes) (back yes)) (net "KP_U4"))
 (via (at 30.900000 30.800000) (size 0.6) (drill 0.3) (layers "F.Cu" "B.Cu") (tenting (front yes) (back yes)) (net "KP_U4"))
 (via (at 31.700000 37.100000) (size 0.6) (drill 0.3) (layers "F.Cu" "B.Cu") (tenting (front yes) (back yes)) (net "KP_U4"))
 (via (at 31.700000 41.800000) (size 0.6) (drill 0.3) (layers "F.Cu" "B.Cu") (tenting (front yes) (back yes)) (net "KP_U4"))
 (segment (start 37.700000 38.000000) (end 35.700000 36.000000) (width 0.508) (layer "F.Cu") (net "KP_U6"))
 (segment (start 35.700000 36.000000) (end 26.200000 36.000000) (width 0.508) (layer "F.Cu") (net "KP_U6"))
 (segment (start 26.200000 36.000000) (end 26.200000 33.800000) (width 0.508) (layer "B.Cu") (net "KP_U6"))
 (segment (start 26.200000 33.800000) (end 26.000000 33.600000) (width 0.508) (layer "F.Cu") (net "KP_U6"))
 (segment (start 26.000000 33.600000) (end 16.800000 33.600000) (width 0.508) (layer "F.Cu") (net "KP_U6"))
 (segment (start 16.800000 33.600000) (end 16.850000 33.625000) (width 0.508) (layer "F.Cu") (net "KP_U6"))
 (segment (start 34.000000 36.000000) (end 34.000000 32.200000) (width 0.508) (layer "B.Cu") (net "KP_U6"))
 (segment (start 34.000000 32.200000) (end 35.100000 31.100000) (width 0.508) (layer "B.Cu") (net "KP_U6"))
 (segment (start 35.100000 31.100000) (end 37.700000 28.500000) (width 0.508) (layer "F.Cu") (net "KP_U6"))
 (segment (start 37.700000 28.500000) (end 37.700000 28.000000) (width 0.508) (layer "F.Cu") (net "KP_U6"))
 (segment (start 37.700000 28.000000) (end 37.700000 20.000000) (width 0.508) (layer "F.Cu") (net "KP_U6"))
 (segment (start 37.700000 38.000000) (end 37.700000 38.500000) (width 0.508) (layer "F.Cu") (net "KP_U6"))
 (segment (start 37.700000 38.500000) (end 37.700000 46.000000) (width 0.508) (layer "B.Cu") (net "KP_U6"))
 (via (at 26.200000 36.000000) (size 0.6) (drill 0.3) (layers "F.Cu" "B.Cu") (tenting (front yes) (back yes)) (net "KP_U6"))
 (via (at 26.200000 33.800000) (size 0.6) (drill 0.3) (layers "F.Cu" "B.Cu") (tenting (front yes) (back yes)) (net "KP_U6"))
 (via (at 34.000000 36.000000) (size 0.6) (drill 0.3) (layers "F.Cu" "B.Cu") (tenting (front yes) (back yes)) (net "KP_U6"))
 (via (at 35.100000 31.100000) (size 0.6) (drill 0.3) (layers "F.Cu" "B.Cu") (tenting (front yes) (back yes)) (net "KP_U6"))
 (via (at 37.700000 38.500000) (size 0.6) (drill 0.3) (layers "F.Cu" "B.Cu") (tenting (front yes) (back yes)) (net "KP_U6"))
 (segment (start 42.780000 38.000000) (end 42.800000 38.000000) (width 0.508) (layer "F.Cu") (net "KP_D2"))
 (segment (start 42.800000 38.000000) (end 40.900000 36.100000) (width 0.508) (layer "F.Cu") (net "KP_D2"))
 (segment (start 40.900000 36.100000) (end 39.800000 36.100000) (width 0.508) (layer "F.Cu") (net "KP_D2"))
 (segment (start 39.800000 36.100000) (end 37.600000 33.900000) (width 0.508) (layer "F.Cu") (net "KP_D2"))
 (segment (start 37.600000 33.900000) (end 37.300000 33.900000) (width 0.508) (layer "F.Cu") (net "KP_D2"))
 (segment (start 37.300000 33.900000) (end 37.200000 33.800000) (width 0.508) (layer "F.Cu") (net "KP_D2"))
 (segment (start 37.200000 33.800000) (end 27.400000 33.800000) (width 0.508) (layer "F.Cu") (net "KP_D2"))
 (segment (start 27.400000 33.800000) (end 27.400000 36.400000) (width 0.508) (layer "B.Cu") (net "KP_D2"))
 (segment (start 27.400000 36.400000) (end 26.600000 37.200000) (width 0.508) (layer "B.Cu") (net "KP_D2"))
 (segment (start 26.600000 37.200000) (end 24.500000 37.200000) (width 0.508) (layer "B.Cu") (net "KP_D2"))
 (segment (start 24.500000 37.200000) (end 23.900000 36.600000) (width 0.508) (layer "B.Cu") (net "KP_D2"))
 (segment (start 23.900000 36.600000) (end 23.400000 36.100000) (width 0.508) (layer "F.Cu") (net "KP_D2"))
 (segment (start 23.400000 36.100000) (end 16.800000 36.100000) (width 0.508) (layer "F.Cu") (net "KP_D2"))
 (segment (start 16.800000 36.100000) (end 16.850000 36.125000) (width 0.508) (layer "F.Cu") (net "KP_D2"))
 (segment (start 38.400000 34.700000) (end 39.100000 34.700000) (width 0.508) (layer "F.Cu") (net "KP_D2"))
 (segment (start 39.100000 34.700000) (end 42.800000 31.000000) (width 0.508) (layer "F.Cu") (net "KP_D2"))
 (segment (start 42.800000 31.000000) (end 42.800000 28.000000) (width 0.508) (layer "F.Cu") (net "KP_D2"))
 (segment (start 42.800000 28.000000) (end 42.780000 28.000000) (width 0.508) (layer "F.Cu") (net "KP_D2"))
 (segment (start 42.800000 28.000000) (end 42.800000 20.000000) (width 0.508) (layer "F.Cu") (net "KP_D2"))
 (segment (start 42.800000 38.000000) (end 42.800000 38.500000) (width 0.508) (layer "F.Cu") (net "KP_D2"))
 (segment (start 42.800000 38.500000) (end 42.800000 46.000000) (width 0.508) (layer "B.Cu") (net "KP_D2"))
 (via (at 27.400000 33.800000) (size 0.6) (drill 0.3) (layers "F.Cu" "B.Cu") (tenting (front yes) (back yes)) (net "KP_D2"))
 (via (at 23.900000 36.600000) (size 0.6) (drill 0.3) (layers "F.Cu" "B.Cu") (tenting (front yes) (back yes)) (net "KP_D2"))
 (via (at 42.800000 38.500000) (size 0.6) (drill 0.3) (layers "F.Cu" "B.Cu") (tenting (front yes) (back yes)) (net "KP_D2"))
 (segment (start 47.860000 38.000000) (end 47.900000 38.000000) (width 0.508) (layer "F.Cu") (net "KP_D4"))
 (segment (start 47.900000 38.000000) (end 47.300000 38.600000) (width 0.508) (layer "F.Cu") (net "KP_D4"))
 (segment (start 47.300000 38.600000) (end 47.000000 38.600000) (width 0.508) (layer "F.Cu") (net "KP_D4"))
 (segment (start 47.000000 38.600000) (end 46.100000 39.500000) (width 0.508) (layer "F.Cu") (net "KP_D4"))
 (segment (start 46.100000 39.500000) (end 45.800000 39.500000) (width 0.508) (layer "F.Cu") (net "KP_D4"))
 (segment (start 45.800000 39.500000) (end 45.700000 39.600000) (width 0.508) (layer "F.Cu") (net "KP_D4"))
 (segment (start 45.700000 39.600000) (end 45.200000 39.600000) (width 0.508) (layer "F.Cu") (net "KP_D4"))
 (segment (start 45.200000 39.600000) (end 44.200000 40.600000) (width 0.508) (layer "F.Cu") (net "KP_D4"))
 (segment (start 44.200000 40.600000) (end 43.900000 40.600000) (width 0.508) (layer "F.Cu") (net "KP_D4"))
 (segment (start 43.900000 40.600000) (end 43.800000 40.700000) (width 0.508) (layer "F.Cu") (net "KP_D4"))
 (segment (start 43.800000 40.700000) (end 18.900000 40.700000) (width 0.508) (layer "F.Cu") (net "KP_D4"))
 (segment (start 18.900000 40.700000) (end 16.800000 38.600000) (width 0.508) (layer "F.Cu") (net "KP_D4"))
 (segment (start 16.800000 38.600000) (end 16.850000 38.625000) (width 0.508) (layer "F.Cu") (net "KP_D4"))
 (segment (start 47.900000 38.000000) (end 47.900000 37.500000) (width 0.508) (layer "F.Cu") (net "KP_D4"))
 (segment (start 47.900000 37.500000) (end 47.900000 35.300000) (width 0.508) (layer "B.Cu") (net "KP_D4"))
 (segment (start 47.900000 35.300000) (end 47.900000 28.000000) (width 0.508) (layer "F.Cu") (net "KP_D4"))
 (segment (start 47.900000 28.000000) (end 47.860000 28.000000) (width 0.508) (layer "F.Cu") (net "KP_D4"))
 (segment (start 47.900000 28.000000) (end 47.900000 20.000000) (width 0.508) (layer "F.Cu") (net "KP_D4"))
 (segment (start 44.200000 40.600000) (end 46.700000 43.100000) (width 0.508) (layer "F.Cu") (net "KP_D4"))
 (segment (start 46.700000 43.100000) (end 45.900000 43.900000) (width 0.508) (layer "F.Cu") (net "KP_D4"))
 (segment (start 45.900000 43.900000) (end 47.900000 45.900000) (width 0.508) (layer "B.Cu") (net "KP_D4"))
 (via (at 47.900000 37.500000) (size 0.6) (drill 0.3) (layers "F.Cu" "B.Cu") (tenting (front yes) (back yes)) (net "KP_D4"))
 (via (at 47.900000 35.300000) (size 0.6) (drill 0.3) (layers "F.Cu" "B.Cu") (tenting (front yes) (back yes)) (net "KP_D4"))
 (via (at 45.900000 43.900000) (size 0.6) (drill 0.3) (layers "F.Cu" "B.Cu") (tenting (front yes) (back yes)) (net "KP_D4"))
 (segment (start 28.400000 37.100000) (end 28.290000 37.250000) (width 0.508) (layer "F.Cu") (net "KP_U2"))
 (segment (start 31.700000 37.100000) (end 31.869999 37.250000) (width 0.508) (layer "F.Cu") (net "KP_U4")))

